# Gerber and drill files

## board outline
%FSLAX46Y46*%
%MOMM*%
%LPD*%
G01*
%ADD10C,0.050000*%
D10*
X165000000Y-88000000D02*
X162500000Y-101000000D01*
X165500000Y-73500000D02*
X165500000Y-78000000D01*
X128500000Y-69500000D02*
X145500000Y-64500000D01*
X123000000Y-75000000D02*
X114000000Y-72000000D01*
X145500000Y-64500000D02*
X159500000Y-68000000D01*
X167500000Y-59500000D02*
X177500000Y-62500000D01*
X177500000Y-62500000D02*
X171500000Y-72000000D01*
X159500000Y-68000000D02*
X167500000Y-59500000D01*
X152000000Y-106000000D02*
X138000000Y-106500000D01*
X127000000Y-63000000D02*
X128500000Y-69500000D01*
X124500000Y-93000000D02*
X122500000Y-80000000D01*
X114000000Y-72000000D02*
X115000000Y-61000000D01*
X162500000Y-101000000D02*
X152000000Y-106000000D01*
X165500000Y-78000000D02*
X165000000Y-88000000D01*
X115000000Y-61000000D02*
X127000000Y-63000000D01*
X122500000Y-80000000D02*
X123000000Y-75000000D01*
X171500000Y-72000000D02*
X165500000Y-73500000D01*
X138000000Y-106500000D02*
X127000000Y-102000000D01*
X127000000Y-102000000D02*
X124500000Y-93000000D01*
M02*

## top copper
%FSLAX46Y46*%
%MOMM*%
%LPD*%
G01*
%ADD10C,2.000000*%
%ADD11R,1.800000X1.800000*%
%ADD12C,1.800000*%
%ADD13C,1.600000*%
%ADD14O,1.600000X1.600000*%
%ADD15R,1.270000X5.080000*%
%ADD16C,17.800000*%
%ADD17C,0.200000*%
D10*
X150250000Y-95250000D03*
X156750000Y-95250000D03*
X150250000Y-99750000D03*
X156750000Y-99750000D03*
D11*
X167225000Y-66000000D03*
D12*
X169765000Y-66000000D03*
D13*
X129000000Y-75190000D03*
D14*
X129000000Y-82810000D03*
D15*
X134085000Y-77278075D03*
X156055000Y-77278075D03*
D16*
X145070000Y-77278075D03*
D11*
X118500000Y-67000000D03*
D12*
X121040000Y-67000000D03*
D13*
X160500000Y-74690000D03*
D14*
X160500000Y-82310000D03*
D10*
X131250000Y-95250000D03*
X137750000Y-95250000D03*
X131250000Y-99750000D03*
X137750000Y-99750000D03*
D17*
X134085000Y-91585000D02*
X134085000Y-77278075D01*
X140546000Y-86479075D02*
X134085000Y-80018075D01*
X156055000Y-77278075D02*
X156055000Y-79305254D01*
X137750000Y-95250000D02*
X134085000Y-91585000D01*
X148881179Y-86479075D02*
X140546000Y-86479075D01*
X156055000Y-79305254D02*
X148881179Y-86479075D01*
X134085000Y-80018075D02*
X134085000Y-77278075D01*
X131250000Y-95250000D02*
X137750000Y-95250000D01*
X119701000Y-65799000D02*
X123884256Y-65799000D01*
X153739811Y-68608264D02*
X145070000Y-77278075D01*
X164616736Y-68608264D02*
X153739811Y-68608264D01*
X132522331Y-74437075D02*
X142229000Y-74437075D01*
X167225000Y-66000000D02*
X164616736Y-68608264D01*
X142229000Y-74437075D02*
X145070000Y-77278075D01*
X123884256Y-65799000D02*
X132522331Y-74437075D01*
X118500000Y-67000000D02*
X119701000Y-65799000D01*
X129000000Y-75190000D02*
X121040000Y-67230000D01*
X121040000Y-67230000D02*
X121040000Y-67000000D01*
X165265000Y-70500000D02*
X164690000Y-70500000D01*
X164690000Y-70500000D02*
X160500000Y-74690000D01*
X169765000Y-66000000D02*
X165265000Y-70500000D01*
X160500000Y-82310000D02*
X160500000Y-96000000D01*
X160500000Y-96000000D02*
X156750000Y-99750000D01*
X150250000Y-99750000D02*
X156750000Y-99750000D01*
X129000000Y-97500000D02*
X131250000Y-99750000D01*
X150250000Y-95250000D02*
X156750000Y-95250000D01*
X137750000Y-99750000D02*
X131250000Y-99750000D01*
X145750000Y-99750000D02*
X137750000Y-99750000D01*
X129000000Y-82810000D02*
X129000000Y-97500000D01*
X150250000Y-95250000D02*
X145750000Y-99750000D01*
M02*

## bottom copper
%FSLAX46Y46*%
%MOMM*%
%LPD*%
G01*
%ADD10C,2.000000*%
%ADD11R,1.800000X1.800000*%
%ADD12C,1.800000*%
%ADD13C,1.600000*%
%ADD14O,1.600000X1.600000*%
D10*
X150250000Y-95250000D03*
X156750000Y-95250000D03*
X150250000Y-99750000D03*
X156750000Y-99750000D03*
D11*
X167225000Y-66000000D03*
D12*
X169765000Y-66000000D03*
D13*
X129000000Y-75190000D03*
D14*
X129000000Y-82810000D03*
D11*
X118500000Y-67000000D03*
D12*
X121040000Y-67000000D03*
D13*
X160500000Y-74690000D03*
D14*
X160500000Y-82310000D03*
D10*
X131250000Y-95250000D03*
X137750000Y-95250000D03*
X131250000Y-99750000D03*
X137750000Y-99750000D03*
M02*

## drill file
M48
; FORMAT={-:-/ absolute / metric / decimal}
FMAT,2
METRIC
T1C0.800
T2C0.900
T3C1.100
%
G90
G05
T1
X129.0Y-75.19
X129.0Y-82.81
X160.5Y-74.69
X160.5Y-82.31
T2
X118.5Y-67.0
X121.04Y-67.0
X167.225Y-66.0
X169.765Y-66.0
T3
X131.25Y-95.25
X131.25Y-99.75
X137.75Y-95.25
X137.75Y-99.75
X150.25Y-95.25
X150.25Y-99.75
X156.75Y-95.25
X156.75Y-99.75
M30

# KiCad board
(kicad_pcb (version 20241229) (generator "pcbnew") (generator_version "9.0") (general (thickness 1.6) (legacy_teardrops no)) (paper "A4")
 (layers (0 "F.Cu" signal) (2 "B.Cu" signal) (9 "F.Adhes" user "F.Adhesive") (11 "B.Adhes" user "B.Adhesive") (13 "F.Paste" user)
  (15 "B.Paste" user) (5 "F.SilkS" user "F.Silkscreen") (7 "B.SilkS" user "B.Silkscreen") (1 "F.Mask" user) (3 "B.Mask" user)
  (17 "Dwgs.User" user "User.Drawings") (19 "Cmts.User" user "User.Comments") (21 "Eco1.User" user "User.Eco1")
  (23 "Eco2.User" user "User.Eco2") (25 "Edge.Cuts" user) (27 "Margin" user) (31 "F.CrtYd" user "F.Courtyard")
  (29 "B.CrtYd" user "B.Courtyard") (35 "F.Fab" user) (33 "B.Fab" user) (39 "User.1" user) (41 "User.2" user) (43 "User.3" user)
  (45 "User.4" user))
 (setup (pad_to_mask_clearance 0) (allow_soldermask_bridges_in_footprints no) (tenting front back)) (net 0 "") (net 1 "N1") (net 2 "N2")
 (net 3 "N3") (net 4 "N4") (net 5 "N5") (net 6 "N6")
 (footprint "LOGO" (layer "F.Cu") (at 130 88)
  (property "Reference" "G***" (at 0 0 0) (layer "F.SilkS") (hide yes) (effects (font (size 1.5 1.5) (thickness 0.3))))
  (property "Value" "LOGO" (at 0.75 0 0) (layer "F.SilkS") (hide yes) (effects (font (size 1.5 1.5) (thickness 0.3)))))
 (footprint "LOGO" (layer "F.Cu") (at 144 94)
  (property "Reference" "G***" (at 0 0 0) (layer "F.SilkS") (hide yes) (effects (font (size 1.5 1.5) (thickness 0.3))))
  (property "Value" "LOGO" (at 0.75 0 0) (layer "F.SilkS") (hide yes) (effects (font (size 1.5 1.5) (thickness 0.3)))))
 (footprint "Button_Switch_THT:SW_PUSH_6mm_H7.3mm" (layer "F.Cu") (at 150.25 95.25)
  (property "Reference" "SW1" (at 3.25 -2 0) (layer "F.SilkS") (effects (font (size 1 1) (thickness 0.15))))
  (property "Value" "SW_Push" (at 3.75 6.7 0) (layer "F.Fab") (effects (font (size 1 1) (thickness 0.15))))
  (pad "1" thru_hole circle (at 0 0 90) (size 2 2) (drill 1.1) (layers "*.Cu" "*.Mask") (remove_unused_layers no) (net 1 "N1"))
  (pad "1" thru_hole circle (at 6.5 0 90) (size 2 2) (drill 1.1) (layers "*.Cu" "*.Mask") (remove_unused_layers no) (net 1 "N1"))
  (pad "2" thru_hole circle (at 0 4.5 90) (size 2 2) (drill 1.1) (layers "*.Cu" "*.Mask") (remove_unused_layers no) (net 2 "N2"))
  (pad "2" thru_hole circle (at 6.5 4.5 90) (size 2 2) (drill 1.1) (layers "*.Cu" "*.Mask") (remove_unused_layers no) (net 2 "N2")))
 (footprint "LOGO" (layer "F.Cu") (at 144 101.5)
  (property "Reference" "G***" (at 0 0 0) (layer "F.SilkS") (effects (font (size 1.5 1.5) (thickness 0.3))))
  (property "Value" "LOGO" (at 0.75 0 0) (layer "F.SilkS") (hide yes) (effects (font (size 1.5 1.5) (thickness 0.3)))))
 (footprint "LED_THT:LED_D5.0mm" (layer "F.Cu") (at 167.225 66)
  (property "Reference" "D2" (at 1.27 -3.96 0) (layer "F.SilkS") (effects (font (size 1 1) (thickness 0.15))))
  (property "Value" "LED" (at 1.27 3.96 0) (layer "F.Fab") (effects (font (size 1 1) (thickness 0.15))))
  (pad "1" thru_hole rect (at 0 0) (size 1.8 1.8) (drill 0.9) (layers "*.Cu" "*.Mask") (remove_unused_layers no) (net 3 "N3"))
  (pad "2" thru_hole circle (at 2.54 0) (size 1.8 1.8) (drill 0.9) (layers "*.Cu" "*.Mask") (remove_unused_layers no) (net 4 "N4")))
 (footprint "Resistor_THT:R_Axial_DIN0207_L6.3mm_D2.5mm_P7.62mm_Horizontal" (layer "F.Cu") (at 129 75.19 -90)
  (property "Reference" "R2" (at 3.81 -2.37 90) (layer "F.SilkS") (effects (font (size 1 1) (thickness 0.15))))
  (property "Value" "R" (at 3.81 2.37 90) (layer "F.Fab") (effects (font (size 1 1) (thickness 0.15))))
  (pad "1" thru_hole circle (at 0 0 270) (size 1.6 1.6) (drill 0.8) (layers "*.Cu" "*.Mask") (remove_unused_layers no) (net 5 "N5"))
  (pad "2" thru_hole oval (at 7.62 0 270) (size 1.6 1.6) (drill 0.8) (layers "*.Cu" "*.Mask") (remove_unused_layers no) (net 1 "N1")))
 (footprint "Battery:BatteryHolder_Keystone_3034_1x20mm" (layer "F.Cu") (at 145.07 77.278075)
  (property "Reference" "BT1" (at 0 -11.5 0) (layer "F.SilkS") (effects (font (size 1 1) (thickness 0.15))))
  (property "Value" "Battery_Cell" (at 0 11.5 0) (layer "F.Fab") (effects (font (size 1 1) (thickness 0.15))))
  (pad "1" smd rect (at -10.985 0) (size 1.27 5.08) (layers "F.Cu" "F.Mask" "F.Paste") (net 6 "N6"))
  (pad "1" smd rect (at 10.985 0) (size 1.27 5.08) (layers "F.Cu" "F.Mask" "F.Paste") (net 6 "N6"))
  (pad "2" smd circle (at 0 0) (size 17.8 17.8) (layers "F.Cu" "F.Mask") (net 3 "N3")))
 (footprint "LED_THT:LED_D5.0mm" (layer "F.Cu") (at 118.5 67)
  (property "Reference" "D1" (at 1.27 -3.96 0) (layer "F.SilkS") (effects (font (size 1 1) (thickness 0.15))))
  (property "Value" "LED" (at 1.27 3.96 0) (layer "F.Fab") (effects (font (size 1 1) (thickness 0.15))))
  (pad "1" thru_hole rect (at 0 0) (size 1.8 1.8) (drill 0.9) (layers "*.Cu" "*.Mask") (remove_unused_layers no) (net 3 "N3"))
  (pad "2" thru_hole circle (at 2.54 0) (size 1.8 1.8) (drill 0.9) (layers "*.Cu" "*.Mask") (remove_unused_layers no) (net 5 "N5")))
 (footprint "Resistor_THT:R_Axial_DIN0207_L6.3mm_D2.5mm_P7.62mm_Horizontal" (layer "F.Cu") (at 160.5 74.69 -90)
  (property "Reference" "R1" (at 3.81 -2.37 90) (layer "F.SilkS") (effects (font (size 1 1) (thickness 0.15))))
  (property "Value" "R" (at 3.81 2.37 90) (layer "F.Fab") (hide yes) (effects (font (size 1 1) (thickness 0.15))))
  (pad "1" thru_hole circle (at 0 0 270) (size 1.6 1.6) (drill 0.8) (layers "*.Cu" "*.Mask") (remove_unused_layers no) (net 4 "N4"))
  (pad "2" thru_hole oval (at 7.62 0 270) (size 1.6 1.6) (drill 0.8) (layers "*.Cu" "*.Mask") (remove_unused_layers no) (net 2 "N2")))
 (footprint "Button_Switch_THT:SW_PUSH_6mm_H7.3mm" (layer "F.Cu") (at 131.25 95.25)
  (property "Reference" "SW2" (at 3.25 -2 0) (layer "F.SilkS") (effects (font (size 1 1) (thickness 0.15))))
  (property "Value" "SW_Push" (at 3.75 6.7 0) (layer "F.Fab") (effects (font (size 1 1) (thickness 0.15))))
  (pad "1" thru_hole circle (at 0 0 90) (size 2 2) (drill 1.1) (layers "*.Cu" "*.Mask") (remove_unused_layers no) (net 6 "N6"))
  (pad "1" thru_hole circle (at 6.5 0 90) (size 2 2) (drill 1.1) (layers "*.Cu" "*.Mask") (remove_unused_layers no) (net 6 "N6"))
  (pad "2" thru_hole circle (at 0 4.5 90) (size 2 2) (drill 1.1) (layers "*.Cu" "*.Mask") (remove_unused_layers no) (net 1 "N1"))
  (pad "2" thru_hole circle (at 6.5 4.5 90) (size 2 2) (drill 1.1) (layers "*.Cu" "*.Mask") (remove_unused_layers no) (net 1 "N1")))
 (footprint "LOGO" (layer "F.Cu") (at 157 88)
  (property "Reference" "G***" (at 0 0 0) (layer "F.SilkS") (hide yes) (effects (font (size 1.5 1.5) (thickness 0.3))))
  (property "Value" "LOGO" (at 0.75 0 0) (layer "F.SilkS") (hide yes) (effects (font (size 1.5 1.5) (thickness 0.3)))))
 (gr_line (start 165 88) (end 162.5 101) (stroke (width 0.05) (type default)) (layer "Edge.Cuts"))
 (gr_line (start 165.5 73.5) (end 165.5 78) (stroke (width 0.05) (type default)) (layer "Edge.Cuts"))
 (gr_line (start 128.5 69.5) (end 145.5 64.5) (stroke (width 0.05) (type default)) (layer "Edge.Cuts"))
 (gr_line (start 123 75) (end 114 72) (stroke (width 0.05) (type default)) (layer "Edge.Cuts"))
 (gr_line (start 145.5 64.5) (end 159.5 68) (stroke (width 0.05) (type default)) (layer "Edge.Cuts"))
 (gr_line (start 167.5 59.5) (end 177.5 62.5) (stroke (width 0.05) (type default)) (layer "Edge.Cuts"))
 (gr_line (start 177.5 62.5) (end 171.5 72) (stroke (width 0.05) (type default)) (layer "Edge.Cuts"))
 (gr_line (start 159.5 68) (end 167.5 59.5) (stroke (width 0.05) (type default)) (layer "Edge.Cuts"))
 (gr_line (start 152 106) (end 138 106.5) (stroke (width 0.05) (type default)) (layer "Edge.Cuts"))
 (gr_line (start 127 63) (end 128.5 69.5) (stroke (width 0.05) (type default)) (layer "Edge.Cuts"))
 (gr_line (start 124.5 93) (end 122.5 80) (stroke (width 0.05) (type default)) (layer "Edge.Cuts"))
 (gr_line (start 114 72) (end 115 61) (stroke (width 0.05) (type default)) (layer "Edge.Cuts"))
 (gr_line (start 162.5 101) (end 152 106) (stroke (width 0.05) (type default)) (layer "Edge.Cuts"))
 (gr_line (start 165.5 78) (end 165 88) (stroke (width 0.05) (type default)) (layer "Edge.Cuts"))
 (gr_line (start 115 61) (end 127 63) (stroke (width 0.05) (type default)) (layer "Edge.Cuts"))
 (gr_line (start 122.5 80) (end 123 75) (stroke (width 0.05) (type default)) (layer "Edge.Cuts"))
 (gr_line (start 171.5 72) (end 165.5 73.5) (stroke (width 0.05) (type default)) (layer "Edge.Cuts"))
 (gr_line (start 138 106.5) (end 127 102) (stroke (width 0.05) (type default)) (layer "Edge.Cuts"))
 (gr_line (start 127 102) (end 124.5 93) (stroke (width 0.05) (type default)) (layer "Edge.Cuts"))
 (segment (start 134.085 91.585) (end 134.085 77.278075) (width 0.2) (layer "F.Cu") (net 6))
 (segment (start 140.546 86.479075) (end 134.085 80.018075) (width 0.2) (layer "F.Cu") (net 6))
 (segment (start 156.055 77.278075) (end 156.055 79.305254) (width 0.2) (layer "F.Cu") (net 6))
 (segment (start 137.75 95.25) (end 134.085 91.585) (width 0.2) (layer "F.Cu") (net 6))
 (segment (start 148.881179 86.479075) (end 140.546 86.479075) (width 0.2) (layer "F.Cu") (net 6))
 (segment (start 156.055 79.305254) (end 148.881179 86.479075) (width 0.2) (layer "F.Cu") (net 6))
 (segment (start 134.085 80.018075) (end 134.085 77.278075) (width 0.2) (layer "F.Cu") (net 6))
 (segment (start 131.25 95.25) (end 137.75 95.25) (width 0.2) (layer "F.Cu") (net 6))
 (segment (start 119.701 65.799) (end 123.884256 65.799) (width 0.2) (layer "F.Cu") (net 3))
 (segment (start 153.739811 68.608264) (end 145.07 77.278075) (width 0.2) (layer "F.Cu") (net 3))
 (segment (start 164.616736 68.608264) (end 153.739811 68.608264) (width 0.2) (layer "F.Cu") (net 3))
 (segment (start 132.522331 74.437075) (end 142.229 74.437075) (width 0.2) (layer "F.Cu") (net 3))
 (segment (start 167.225 66) (end 164.616736 68.608264) (width 0.2) (layer "F.Cu") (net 3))
 (segment (start 142.229 74.437075) (end 145.07 77.278075) (width 0.2) (layer "F.Cu") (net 3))
 (segment (start 123.884256 65.799) (end 132.522331 74.437075) (width 0.2) (layer "F.Cu") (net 3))
 (segment (start 118.5 67) (end 119.701 65.799) (width 0.2) (layer "F.Cu") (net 3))
 (segment (start 129 75.19) (end 121.04 67.23) (width 0.2) (layer "F.Cu") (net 5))
 (segment (start 121.04 67.23) (end 121.04 67) (width 0.2) (layer "F.Cu") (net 5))
 (segment (start 165.265 70.5) (end 164.69 70.5) (width 0.2) (layer "F.Cu") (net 4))
 (segment (start 164.69 70.5) (end 160.5 74.69) (width 0.2) (layer "F.Cu") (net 4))
 (segment (start 169.765 66) (end 165.265 70.5) (width 0.2) (layer "F.Cu") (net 4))
 (segment (start 160.5 82.31) (end 160.5 96) (width 0.2) (layer "F.Cu") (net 2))
 (segment (start 160.5 96) (end 156.75 99.75) (width 0.2) (layer "F.Cu") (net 2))
 (segment (start 150.25 99.75) (end 156.75 99.75) (width 0.2) (layer "F.Cu") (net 2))
 (segment (start 129 97.5) (end 131.25 99.75) (width 0.2) (layer "F.Cu") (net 1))
 (segment (start 150.25 95.25) (end 156.75 95.25) (width 0.2) (layer "F.Cu") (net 1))
 (segment (start 137.75 99.75) (end 131.25 99.75) (width 0.2) (layer "F.Cu") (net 1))
 (segment (start 145.75 99.75) (end 137.75 99.75) (width 0.2) (layer "F.Cu") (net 1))
 (segment (start 129 82.81) (end 129 97.5) (width 0.2) (layer "F.Cu") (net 1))
 (segment (start 150.25 95.25) (end 145.75 99.75) (width 0.2) (layer "F.Cu") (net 1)))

